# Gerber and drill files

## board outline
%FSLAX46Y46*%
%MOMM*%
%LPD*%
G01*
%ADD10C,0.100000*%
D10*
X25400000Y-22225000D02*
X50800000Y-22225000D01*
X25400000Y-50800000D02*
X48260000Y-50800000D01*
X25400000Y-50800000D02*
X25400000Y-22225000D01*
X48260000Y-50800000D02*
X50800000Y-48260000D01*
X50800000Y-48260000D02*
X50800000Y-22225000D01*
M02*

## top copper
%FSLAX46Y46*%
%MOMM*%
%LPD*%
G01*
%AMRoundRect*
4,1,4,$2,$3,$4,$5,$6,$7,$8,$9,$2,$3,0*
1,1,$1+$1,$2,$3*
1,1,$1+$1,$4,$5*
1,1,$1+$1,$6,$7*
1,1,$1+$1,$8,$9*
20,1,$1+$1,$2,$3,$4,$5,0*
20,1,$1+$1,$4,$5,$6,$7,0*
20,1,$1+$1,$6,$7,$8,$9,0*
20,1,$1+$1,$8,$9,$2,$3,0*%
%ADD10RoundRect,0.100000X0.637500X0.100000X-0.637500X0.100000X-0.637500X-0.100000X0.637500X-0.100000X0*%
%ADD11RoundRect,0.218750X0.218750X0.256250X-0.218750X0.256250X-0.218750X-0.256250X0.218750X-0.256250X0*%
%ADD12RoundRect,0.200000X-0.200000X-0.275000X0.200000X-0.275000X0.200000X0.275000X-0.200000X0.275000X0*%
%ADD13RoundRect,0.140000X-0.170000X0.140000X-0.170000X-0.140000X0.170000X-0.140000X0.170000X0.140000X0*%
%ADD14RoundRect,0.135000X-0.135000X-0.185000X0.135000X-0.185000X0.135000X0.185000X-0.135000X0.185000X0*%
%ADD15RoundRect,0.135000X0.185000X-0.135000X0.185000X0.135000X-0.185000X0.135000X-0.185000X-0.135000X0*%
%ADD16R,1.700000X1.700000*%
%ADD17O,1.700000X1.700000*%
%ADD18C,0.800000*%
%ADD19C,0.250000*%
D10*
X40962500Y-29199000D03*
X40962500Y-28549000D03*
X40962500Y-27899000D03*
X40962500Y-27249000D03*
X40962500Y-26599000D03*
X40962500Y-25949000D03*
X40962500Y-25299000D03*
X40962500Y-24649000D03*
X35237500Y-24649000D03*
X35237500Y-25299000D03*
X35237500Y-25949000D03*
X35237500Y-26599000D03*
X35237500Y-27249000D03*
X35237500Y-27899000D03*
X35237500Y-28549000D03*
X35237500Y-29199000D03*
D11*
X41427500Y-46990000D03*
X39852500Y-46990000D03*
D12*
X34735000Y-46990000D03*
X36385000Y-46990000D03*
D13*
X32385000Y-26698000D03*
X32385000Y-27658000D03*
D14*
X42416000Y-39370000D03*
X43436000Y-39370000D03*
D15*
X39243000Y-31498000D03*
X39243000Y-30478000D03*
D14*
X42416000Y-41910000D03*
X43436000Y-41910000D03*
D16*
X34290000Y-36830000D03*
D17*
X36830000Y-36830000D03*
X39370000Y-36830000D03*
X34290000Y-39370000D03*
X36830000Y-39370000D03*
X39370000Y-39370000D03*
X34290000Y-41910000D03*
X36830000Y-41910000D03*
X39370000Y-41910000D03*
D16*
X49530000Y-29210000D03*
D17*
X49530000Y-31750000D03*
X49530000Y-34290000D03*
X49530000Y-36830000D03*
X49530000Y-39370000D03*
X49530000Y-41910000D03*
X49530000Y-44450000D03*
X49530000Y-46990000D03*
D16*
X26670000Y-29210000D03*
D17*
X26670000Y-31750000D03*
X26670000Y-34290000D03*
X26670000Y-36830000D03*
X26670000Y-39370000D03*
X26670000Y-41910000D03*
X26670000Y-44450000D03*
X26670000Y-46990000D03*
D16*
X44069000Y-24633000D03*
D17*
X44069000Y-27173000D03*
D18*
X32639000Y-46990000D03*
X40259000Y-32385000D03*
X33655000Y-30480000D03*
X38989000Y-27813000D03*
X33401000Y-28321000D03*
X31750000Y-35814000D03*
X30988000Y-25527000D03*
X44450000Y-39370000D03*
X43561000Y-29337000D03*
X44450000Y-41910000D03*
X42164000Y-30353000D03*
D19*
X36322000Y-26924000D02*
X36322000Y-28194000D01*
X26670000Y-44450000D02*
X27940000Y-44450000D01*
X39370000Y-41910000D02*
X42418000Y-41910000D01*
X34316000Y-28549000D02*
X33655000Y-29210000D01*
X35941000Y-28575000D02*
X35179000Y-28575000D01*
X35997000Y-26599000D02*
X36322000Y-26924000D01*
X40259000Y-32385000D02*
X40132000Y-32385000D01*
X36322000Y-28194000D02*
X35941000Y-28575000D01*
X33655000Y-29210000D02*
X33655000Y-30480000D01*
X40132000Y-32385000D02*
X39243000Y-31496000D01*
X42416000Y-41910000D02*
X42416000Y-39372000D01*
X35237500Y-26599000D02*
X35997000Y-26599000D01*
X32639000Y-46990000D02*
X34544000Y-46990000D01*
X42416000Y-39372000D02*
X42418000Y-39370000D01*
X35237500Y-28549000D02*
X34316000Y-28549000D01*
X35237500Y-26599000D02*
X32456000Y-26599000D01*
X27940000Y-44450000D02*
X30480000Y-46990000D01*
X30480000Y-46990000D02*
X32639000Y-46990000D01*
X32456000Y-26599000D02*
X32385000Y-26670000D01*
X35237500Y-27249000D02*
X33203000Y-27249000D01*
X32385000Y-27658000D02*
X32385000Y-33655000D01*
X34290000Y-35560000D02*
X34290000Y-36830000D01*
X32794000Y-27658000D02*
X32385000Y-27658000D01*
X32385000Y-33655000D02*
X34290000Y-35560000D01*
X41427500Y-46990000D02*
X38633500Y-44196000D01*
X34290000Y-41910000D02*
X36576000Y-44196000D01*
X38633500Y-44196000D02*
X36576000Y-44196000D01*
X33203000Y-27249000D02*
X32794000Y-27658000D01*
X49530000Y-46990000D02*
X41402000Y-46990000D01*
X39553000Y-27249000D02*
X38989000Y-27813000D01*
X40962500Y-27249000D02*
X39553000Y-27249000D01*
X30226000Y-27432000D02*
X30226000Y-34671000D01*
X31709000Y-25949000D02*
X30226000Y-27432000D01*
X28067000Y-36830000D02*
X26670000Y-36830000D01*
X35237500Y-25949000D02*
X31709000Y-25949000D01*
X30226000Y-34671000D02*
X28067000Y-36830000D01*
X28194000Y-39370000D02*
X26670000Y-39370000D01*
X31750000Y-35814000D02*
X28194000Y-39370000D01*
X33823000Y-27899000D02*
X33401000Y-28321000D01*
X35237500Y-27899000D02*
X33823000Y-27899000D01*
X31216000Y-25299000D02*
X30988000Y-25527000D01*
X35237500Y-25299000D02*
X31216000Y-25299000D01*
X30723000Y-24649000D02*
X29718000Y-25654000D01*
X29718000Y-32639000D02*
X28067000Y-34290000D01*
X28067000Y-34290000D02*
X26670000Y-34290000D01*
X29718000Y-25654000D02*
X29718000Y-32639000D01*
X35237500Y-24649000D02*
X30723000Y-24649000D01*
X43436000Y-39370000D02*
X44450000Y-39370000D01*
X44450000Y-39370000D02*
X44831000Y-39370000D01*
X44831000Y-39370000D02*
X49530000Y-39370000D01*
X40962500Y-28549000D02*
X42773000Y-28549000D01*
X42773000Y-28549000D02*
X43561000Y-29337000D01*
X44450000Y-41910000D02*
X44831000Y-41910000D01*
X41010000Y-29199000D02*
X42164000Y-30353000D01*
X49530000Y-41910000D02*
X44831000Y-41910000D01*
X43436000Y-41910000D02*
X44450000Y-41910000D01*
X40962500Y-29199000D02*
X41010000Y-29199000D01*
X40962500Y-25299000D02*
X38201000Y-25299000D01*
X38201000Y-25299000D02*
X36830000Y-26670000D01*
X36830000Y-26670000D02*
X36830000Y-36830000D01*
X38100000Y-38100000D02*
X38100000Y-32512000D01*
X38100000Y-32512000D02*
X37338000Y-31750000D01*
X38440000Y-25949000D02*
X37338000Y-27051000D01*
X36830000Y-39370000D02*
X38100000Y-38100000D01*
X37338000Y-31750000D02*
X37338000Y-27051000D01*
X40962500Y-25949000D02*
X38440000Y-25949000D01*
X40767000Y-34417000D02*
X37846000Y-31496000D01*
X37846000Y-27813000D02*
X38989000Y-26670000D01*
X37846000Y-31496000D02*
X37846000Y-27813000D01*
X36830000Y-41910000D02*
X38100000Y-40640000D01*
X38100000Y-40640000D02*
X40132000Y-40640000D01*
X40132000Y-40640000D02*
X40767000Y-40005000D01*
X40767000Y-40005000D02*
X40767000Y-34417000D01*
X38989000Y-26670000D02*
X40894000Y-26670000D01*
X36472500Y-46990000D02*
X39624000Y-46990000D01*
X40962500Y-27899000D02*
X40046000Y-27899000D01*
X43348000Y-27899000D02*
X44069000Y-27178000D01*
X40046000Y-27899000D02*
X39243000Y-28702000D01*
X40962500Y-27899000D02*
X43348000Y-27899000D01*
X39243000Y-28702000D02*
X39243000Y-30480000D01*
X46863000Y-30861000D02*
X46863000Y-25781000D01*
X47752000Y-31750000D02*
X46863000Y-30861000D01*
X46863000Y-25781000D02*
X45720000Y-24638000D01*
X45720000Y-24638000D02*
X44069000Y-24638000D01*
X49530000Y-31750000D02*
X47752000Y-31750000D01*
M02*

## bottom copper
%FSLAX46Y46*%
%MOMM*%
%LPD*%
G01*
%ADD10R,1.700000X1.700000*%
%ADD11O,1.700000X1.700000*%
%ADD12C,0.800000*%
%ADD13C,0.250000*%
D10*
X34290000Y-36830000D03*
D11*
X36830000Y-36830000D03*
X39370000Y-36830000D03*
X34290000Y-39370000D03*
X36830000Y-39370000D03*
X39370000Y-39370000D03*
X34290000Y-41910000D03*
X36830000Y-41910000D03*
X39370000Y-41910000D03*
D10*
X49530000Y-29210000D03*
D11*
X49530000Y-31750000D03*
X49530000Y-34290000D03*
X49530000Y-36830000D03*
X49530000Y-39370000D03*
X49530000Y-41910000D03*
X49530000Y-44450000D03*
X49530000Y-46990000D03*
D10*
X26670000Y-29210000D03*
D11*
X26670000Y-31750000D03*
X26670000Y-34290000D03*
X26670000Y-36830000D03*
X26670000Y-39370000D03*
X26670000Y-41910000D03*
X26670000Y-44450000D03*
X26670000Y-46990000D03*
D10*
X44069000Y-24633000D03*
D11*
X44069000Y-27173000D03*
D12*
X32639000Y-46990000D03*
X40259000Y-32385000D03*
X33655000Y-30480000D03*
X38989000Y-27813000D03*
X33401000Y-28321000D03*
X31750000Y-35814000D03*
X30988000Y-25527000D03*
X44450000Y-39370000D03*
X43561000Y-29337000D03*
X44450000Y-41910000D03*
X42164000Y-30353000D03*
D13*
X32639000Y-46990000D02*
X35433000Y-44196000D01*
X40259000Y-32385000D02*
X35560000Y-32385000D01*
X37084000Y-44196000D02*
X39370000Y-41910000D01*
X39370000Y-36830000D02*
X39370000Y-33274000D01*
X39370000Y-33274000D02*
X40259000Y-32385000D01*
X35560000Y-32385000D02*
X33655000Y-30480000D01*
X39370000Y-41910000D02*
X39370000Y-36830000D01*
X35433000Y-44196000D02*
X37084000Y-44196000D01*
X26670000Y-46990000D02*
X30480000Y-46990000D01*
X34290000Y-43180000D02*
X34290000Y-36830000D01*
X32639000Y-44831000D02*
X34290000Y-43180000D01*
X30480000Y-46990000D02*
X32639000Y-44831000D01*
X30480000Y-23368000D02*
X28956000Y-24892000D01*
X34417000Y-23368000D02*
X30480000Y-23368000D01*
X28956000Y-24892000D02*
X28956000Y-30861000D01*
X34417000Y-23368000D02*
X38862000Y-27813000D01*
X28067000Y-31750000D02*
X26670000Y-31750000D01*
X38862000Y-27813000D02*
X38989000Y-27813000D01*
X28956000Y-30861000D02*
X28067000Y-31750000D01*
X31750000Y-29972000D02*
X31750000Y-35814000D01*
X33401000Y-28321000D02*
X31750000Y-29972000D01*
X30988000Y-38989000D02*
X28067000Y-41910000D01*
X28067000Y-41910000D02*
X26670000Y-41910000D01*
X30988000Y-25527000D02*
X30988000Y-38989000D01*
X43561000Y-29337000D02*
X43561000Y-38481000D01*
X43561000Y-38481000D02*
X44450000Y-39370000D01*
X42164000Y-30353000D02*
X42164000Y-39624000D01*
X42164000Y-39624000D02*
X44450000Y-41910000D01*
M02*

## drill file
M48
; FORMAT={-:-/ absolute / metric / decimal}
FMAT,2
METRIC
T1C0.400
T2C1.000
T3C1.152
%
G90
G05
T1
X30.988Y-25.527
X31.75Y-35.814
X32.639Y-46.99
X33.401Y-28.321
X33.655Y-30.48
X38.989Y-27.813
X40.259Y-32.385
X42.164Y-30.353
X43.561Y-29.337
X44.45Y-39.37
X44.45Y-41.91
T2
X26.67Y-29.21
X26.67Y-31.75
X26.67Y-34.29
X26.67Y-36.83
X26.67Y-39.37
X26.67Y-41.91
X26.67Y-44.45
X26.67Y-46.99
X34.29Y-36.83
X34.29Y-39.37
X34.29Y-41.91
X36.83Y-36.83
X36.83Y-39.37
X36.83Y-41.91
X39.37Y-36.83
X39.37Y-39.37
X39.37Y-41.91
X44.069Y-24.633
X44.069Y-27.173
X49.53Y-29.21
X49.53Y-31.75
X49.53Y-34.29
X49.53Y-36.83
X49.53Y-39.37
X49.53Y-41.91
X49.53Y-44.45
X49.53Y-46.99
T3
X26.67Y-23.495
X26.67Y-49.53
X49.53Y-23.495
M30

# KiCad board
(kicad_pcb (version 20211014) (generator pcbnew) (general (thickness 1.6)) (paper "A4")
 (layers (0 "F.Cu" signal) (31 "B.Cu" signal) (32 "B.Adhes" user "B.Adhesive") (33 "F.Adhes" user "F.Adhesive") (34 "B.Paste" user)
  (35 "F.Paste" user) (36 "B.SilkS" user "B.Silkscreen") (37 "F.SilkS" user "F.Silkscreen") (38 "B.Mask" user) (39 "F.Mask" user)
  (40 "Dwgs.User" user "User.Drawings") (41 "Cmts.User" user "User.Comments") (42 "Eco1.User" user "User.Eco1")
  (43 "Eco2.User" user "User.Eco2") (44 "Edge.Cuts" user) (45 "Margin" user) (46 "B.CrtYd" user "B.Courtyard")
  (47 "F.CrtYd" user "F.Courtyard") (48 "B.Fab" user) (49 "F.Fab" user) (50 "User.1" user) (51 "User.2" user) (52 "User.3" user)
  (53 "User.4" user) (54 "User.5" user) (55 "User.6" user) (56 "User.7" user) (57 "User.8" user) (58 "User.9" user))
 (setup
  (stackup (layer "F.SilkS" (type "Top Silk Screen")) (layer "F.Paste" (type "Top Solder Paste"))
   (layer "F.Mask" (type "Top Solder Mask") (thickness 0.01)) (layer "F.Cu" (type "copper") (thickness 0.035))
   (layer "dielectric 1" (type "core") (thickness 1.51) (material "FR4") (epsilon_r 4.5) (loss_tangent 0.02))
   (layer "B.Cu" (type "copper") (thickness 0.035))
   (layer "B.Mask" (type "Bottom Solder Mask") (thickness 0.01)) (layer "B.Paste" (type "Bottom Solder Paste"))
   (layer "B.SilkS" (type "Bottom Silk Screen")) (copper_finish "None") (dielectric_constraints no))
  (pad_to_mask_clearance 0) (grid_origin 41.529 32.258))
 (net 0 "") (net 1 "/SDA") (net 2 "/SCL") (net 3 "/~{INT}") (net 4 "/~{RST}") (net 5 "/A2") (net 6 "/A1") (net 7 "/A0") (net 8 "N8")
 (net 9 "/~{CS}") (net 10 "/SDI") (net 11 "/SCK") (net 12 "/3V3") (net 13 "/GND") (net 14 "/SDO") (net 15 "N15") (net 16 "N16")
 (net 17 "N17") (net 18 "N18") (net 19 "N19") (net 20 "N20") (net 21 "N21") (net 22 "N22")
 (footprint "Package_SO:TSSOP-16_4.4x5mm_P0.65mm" (layer "F.Cu") (at 38.1 26.924 180)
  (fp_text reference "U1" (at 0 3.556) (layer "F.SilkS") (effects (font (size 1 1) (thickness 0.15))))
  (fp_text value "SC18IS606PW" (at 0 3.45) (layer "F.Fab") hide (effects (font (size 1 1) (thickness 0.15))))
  (pad "1" smd roundrect (at -2.8625 -2.275 180) (size 1.475 0.4) (layers "F.Cu" "F.Paste" "F.Mask") (roundrect_rratio 0.25) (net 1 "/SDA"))
  (pad "2" smd roundrect (at -2.8625 -1.625 180) (size 1.475 0.4) (layers "F.Cu" "F.Paste" "F.Mask") (roundrect_rratio 0.25) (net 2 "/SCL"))
  (pad "3" smd roundrect (at -2.8625 -0.975 180) (size 1.475 0.4) (layers "F.Cu" "F.Paste" "F.Mask") (roundrect_rratio 0.25)
   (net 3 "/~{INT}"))
  (pad "4" smd roundrect (at -2.8625 -0.325 180) (size 1.475 0.4) (layers "F.Cu" "F.Paste" "F.Mask") (roundrect_rratio 0.25)
   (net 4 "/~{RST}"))
  (pad "5" smd roundrect (at -2.8625 0.325 180) (size 1.475 0.4) (layers "F.Cu" "F.Paste" "F.Mask") (roundrect_rratio 0.25) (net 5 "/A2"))
  (pad "6" smd roundrect (at -2.8625 0.975 180) (size 1.475 0.4) (layers "F.Cu" "F.Paste" "F.Mask") (roundrect_rratio 0.25) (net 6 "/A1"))
  (pad "7" smd roundrect (at -2.8625 1.625 180) (size 1.475 0.4) (layers "F.Cu" "F.Paste" "F.Mask") (roundrect_rratio 0.25) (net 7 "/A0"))
  (pad "8" smd roundrect (at -2.8625 2.275 180) (size 1.475 0.4) (layers "F.Cu" "F.Paste" "F.Mask") (roundrect_rratio 0.25) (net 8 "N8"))
  (pad "9" smd roundrect (at 2.8625 2.275 180) (size 1.475 0.4) (layers "F.Cu" "F.Paste" "F.Mask") (roundrect_rratio 0.25) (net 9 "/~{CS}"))
  (pad "10" smd roundrect (at 2.8625 1.625 180) (size 1.475 0.4) (layers "F.Cu" "F.Paste" "F.Mask") (roundrect_rratio 0.25) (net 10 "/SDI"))
  (pad "11" smd roundrect (at 2.8625 0.975 180) (size 1.475 0.4) (layers "F.Cu" "F.Paste" "F.Mask") (roundrect_rratio 0.25) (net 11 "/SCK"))
  (pad "12" smd roundrect (at 2.8625 0.325 180) (size 1.475 0.4) (layers "F.Cu" "F.Paste" "F.Mask") (roundrect_rratio 0.25) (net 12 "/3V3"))
  (pad "13" smd roundrect (at 2.8625 -0.325 180) (size 1.475 0.4) (layers "F.Cu" "F.Paste" "F.Mask") (roundrect_rratio 0.25) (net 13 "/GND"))
  (pad "14" smd roundrect (at 2.8625 -0.975 180) (size 1.475 0.4) (layers "F.Cu" "F.Paste" "F.Mask") (roundrect_rratio 0.25) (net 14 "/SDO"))
  (pad "15" smd roundrect (at 2.8625 -1.625 180) (size 1.475 0.4) (layers "F.Cu" "F.Paste" "F.Mask") (roundrect_rratio 0.25) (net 12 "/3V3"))
  (pad "16" smd roundrect (at 2.8625 -2.275 180) (size 1.475 0.4) (layers "F.Cu" "F.Paste" "F.Mask") (roundrect_rratio 0.25) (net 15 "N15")))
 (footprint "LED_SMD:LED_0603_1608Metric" (layer "F.Cu") (at 40.64 46.99 180)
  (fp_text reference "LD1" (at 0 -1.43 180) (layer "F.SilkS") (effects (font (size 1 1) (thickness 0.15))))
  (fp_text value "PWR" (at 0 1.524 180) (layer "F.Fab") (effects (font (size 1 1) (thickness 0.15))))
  (pad "1" smd roundrect (at -0.7875 0 180) (size 0.875 0.95) (layers "F.Cu" "F.Paste" "F.Mask") (roundrect_rratio 0.25) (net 13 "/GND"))
  (pad "2" smd roundrect (at 0.7875 0 180) (size 0.875 0.95) (layers "F.Cu" "F.Paste" "F.Mask") (roundrect_rratio 0.25) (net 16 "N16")))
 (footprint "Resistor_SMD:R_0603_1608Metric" (layer "F.Cu") (at 35.56 46.99)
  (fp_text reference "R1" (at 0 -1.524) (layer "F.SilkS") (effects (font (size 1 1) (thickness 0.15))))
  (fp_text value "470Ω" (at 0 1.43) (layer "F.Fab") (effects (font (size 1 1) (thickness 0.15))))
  (pad "1" smd roundrect (at -0.825 0) (size 0.8 0.95) (layers "F.Cu" "F.Paste" "F.Mask") (roundrect_rratio 0.25) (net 12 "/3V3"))
  (pad "2" smd roundrect (at 0.825 0) (size 0.8 0.95) (layers "F.Cu" "F.Paste" "F.Mask") (roundrect_rratio 0.25) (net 16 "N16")))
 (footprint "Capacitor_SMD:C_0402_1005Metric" (layer "F.Cu") (at 32.385 27.178 -90)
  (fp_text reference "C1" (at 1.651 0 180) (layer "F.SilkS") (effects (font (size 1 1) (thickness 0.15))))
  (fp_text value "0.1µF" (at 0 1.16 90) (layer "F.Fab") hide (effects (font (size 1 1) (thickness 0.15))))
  (pad "1" smd roundrect (at -0.48 0 270) (size 0.56 0.62) (layers "F.Cu" "F.Paste" "F.Mask") (roundrect_rratio 0.25) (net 12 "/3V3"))
  (pad "2" smd roundrect (at 0.48 0 270) (size 0.56 0.62) (layers "F.Cu" "F.Paste" "F.Mask") (roundrect_rratio 0.25) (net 13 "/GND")))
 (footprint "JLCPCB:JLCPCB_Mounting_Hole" (layer "F.Cu") (at 26.67 23.495)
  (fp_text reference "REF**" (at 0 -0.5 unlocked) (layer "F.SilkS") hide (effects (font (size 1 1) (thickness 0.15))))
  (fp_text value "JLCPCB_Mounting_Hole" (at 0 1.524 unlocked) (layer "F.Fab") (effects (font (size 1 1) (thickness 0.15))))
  (pad "" np_thru_hole circle (at 0 0) (size 1.152 1.152) (drill 1.152) (layers F&B.Cu *.Mask) (solder_mask_margin 0.148)))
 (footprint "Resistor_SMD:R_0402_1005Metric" (layer "F.Cu") (at 42.926 39.37)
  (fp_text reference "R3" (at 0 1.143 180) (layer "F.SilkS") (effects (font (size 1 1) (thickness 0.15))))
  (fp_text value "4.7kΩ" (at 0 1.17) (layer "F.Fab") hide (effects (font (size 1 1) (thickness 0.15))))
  (pad "1" smd roundrect (at -0.51 0) (size 0.54 0.64) (layers "F.Cu" "F.Paste" "F.Mask") (roundrect_rratio 0.25) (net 12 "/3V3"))
  (pad "2" smd roundrect (at 0.51 0) (size 0.54 0.64) (layers "F.Cu" "F.Paste" "F.Mask") (roundrect_rratio 0.25) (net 2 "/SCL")))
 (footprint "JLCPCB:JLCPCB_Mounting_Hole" (layer "F.Cu") (at 26.67 49.53)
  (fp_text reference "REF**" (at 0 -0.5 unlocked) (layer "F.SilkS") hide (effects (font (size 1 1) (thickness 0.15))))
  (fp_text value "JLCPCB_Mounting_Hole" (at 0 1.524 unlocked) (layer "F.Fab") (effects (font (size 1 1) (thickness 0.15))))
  (pad "" np_thru_hole circle (at 0 0) (size 1.152 1.152) (drill 1.152) (layers F&B.Cu *.Mask) (solder_mask_margin 0.148)))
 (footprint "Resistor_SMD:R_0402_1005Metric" (layer "F.Cu") (at 39.243 30.988 90)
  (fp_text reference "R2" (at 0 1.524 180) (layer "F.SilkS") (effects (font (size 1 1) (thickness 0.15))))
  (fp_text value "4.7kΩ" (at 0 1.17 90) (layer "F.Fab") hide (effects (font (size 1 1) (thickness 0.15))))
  (pad "1" smd roundrect (at -0.51 0 90) (size 0.54 0.64) (layers "F.Cu" "F.Paste" "F.Mask") (roundrect_rratio 0.25) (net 12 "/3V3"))
  (pad "2" smd roundrect (at 0.51 0 90) (size 0.54 0.64) (layers "F.Cu" "F.Paste" "F.Mask") (roundrect_rratio 0.25) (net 3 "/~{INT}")))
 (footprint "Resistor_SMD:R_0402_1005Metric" (layer "F.Cu") (at 42.926 41.91)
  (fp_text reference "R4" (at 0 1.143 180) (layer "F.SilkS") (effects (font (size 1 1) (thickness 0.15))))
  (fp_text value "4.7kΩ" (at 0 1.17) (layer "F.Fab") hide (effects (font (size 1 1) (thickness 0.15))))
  (pad "1" smd roundrect (at -0.51 0) (size 0.54 0.64) (layers "F.Cu" "F.Paste" "F.Mask") (roundrect_rratio 0.25) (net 12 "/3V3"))
  (pad "2" smd roundrect (at 0.51 0) (size 0.54 0.64) (layers "F.Cu" "F.Paste" "F.Mask") (roundrect_rratio 0.25) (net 1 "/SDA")))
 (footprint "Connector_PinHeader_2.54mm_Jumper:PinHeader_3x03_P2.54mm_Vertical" (layer "F.Cu") (at 34.29 36.83)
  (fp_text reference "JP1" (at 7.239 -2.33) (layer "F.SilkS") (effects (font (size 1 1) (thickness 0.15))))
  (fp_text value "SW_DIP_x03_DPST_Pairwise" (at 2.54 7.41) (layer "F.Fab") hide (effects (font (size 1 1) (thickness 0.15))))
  (pad "1" thru_hole rect (at 0 0) (size 1.7 1.7) (drill 1) (layers *.Cu *.Mask) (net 13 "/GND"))
  (pad "2" thru_hole oval (at 2.54 0) (size 1.7 1.7) (drill 1) (layers *.Cu *.Mask) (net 7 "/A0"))
  (pad "3" thru_hole oval (at 5.08 0) (size 1.7 1.7) (drill 1) (layers *.Cu *.Mask) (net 12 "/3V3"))
  (pad "4" thru_hole oval (at 0 2.54) (size 1.7 1.7) (drill 1) (layers *.Cu *.Mask) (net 13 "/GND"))
  (pad "5" thru_hole oval (at 2.54 2.54) (size 1.7 1.7) (drill 1) (layers *.Cu *.Mask) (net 6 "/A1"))
  (pad "6" thru_hole oval (at 5.08 2.54) (size 1.7 1.7) (drill 1) (layers *.Cu *.Mask) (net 12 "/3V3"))
  (pad "7" thru_hole oval (at 0 5.08) (size 1.7 1.7) (drill 1) (layers *.Cu *.Mask) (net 13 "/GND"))
  (pad "8" thru_hole oval (at 2.54 5.08) (size 1.7 1.7) (drill 1) (layers *.Cu *.Mask) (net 5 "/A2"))
  (pad "9" thru_hole oval (at 5.08 5.08) (size 1.7 1.7) (drill 1) (layers *.Cu *.Mask) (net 12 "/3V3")))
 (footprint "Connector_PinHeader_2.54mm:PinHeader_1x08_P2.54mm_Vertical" (layer "F.Cu") (at 49.53 29.21)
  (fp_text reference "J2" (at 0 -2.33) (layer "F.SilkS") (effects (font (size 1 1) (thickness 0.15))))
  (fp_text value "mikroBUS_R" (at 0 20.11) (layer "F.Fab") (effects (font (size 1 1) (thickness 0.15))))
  (pad "1" thru_hole rect (at 0 0) (size 1.7 1.7) (drill 1) (layers *.Cu *.Mask) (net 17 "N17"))
  (pad "2" thru_hole oval (at 0 2.54) (size 1.7 1.7) (drill 1) (layers *.Cu *.Mask) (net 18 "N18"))
  (pad "3" thru_hole oval (at 0 5.08) (size 1.7 1.7) (drill 1) (layers *.Cu *.Mask) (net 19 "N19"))
  (pad "4" thru_hole oval (at 0 7.62) (size 1.7 1.7) (drill 1) (layers *.Cu *.Mask) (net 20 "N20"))
  (pad "5" thru_hole oval (at 0 10.16) (size 1.7 1.7) (drill 1) (layers *.Cu *.Mask) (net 2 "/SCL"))
  (pad "6" thru_hole oval (at 0 12.7) (size 1.7 1.7) (drill 1) (layers *.Cu *.Mask) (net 1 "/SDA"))
  (pad "7" thru_hole oval (at 0 15.24) (size 1.7 1.7) (drill 1) (layers *.Cu *.Mask) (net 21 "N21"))
  (pad "8" thru_hole oval (at 0 17.78) (size 1.7 1.7) (drill 1) (layers *.Cu *.Mask) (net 13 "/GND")))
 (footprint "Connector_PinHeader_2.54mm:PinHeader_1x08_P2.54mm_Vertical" (layer "F.Cu") (at 26.67 29.21)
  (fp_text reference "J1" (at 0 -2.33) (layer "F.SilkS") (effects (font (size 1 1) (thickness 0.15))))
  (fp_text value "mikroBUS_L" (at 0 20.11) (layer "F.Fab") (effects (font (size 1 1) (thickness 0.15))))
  (pad "1" thru_hole rect (at 0 0) (size 1.7 1.7) (drill 1) (layers *.Cu *.Mask) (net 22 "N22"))
  (pad "2" thru_hole oval (at 0 2.54) (size 1.7 1.7) (drill 1) (layers *.Cu *.Mask) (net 4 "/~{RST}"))
  (pad "3" thru_hole oval (at 0 5.08) (size 1.7 1.7) (drill 1) (layers *.Cu *.Mask) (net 9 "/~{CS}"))
  (pad "4" thru_hole oval (at 0 7.62) (size 1.7 1.7) (drill 1) (layers *.Cu *.Mask) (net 11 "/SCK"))
  (pad "5" thru_hole oval (at 0 10.16) (size 1.7 1.7) (drill 1) (layers *.Cu *.Mask) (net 14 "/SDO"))
  (pad "6" thru_hole oval (at 0 12.7) (size 1.7 1.7) (drill 1) (layers *.Cu *.Mask) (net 10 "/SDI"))
  (pad "7" thru_hole oval (at 0 15.24) (size 1.7 1.7) (drill 1) (layers *.Cu *.Mask) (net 12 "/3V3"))
  (pad "8" thru_hole oval (at 0 17.78) (size 1.7 1.7) (drill 1) (layers *.Cu *.Mask) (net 13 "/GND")))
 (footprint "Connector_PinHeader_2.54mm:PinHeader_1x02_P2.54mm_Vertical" (layer "F.Cu") (at 44.069 24.633)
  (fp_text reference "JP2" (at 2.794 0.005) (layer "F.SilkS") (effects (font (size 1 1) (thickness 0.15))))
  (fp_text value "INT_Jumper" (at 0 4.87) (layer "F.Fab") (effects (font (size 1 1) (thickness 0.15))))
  (pad "1" thru_hole rect (at 0 0) (size 1.7 1.7) (drill 1) (layers *.Cu *.Mask) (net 18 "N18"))
  (pad "2" thru_hole oval (at 0 2.54) (size 1.7 1.7) (drill 1) (layers *.Cu *.Mask) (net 3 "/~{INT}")))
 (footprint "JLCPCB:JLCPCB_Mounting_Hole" (layer "F.Cu") (at 49.53 23.495)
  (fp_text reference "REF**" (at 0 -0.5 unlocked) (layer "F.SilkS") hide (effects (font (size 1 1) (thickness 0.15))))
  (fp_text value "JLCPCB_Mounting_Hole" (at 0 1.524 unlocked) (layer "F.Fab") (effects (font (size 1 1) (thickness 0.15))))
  (pad "" np_thru_hole circle (at 0 0) (size 1.152 1.152) (drill 1.152) (layers F&B.Cu *.Mask) (solder_mask_margin 0.148)))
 (gr_line (start 25.4 22.225) (end 50.8 22.225) (layer "Edge.Cuts") (width 0.1))
 (gr_line (start 25.4 50.8) (end 48.26 50.8) (layer "Edge.Cuts") (width 0.1))
 (gr_line (start 25.4 50.8) (end 25.4 22.225) (layer "Edge.Cuts") (width 0.1))
 (gr_line (start 48.26 50.8) (end 50.8 48.26) (layer "Edge.Cuts") (width 0.1))
 (gr_line (start 50.8 48.26) (end 50.8 22.225) (layer "Edge.Cuts") (width 0.1))
 (segment (start 36.322 26.924) (end 36.322 28.194) (width 0.25) (layer "F.Cu") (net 12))
 (segment (start 26.67 44.45) (end 27.94 44.45) (width 0.25) (layer "F.Cu") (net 12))
 (segment (start 39.37 41.91) (end 42.418 41.91) (width 0.25) (layer "F.Cu") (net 12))
 (segment (start 34.316 28.549) (end 33.655 29.21) (width 0.25) (layer "F.Cu") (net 12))
 (segment (start 35.941 28.575) (end 35.179 28.575) (width 0.25) (layer "F.Cu") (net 12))
 (segment (start 35.997 26.599) (end 36.322 26.924) (width 0.25) (layer "F.Cu") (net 12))
 (segment (start 40.259 32.385) (end 40.132 32.385) (width 0.25) (layer "F.Cu") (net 12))
 (segment (start 36.322 28.194) (end 35.941 28.575) (width 0.25) (layer "F.Cu") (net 12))
 (segment (start 33.655 29.21) (end 33.655 30.48) (width 0.25) (layer "F.Cu") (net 12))
 (segment (start 40.132 32.385) (end 39.243 31.496) (width 0.25) (layer "F.Cu") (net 12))
 (segment (start 42.416 41.91) (end 42.416 39.372) (width 0.25) (layer "F.Cu") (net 12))
 (segment (start 35.2375 26.599) (end 35.997 26.599) (width 0.25) (layer "F.Cu") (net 12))
 (segment (start 32.639 46.99) (end 34.544 46.99) (width 0.25) (layer "F.Cu") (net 12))
 (segment (start 42.416 39.372) (end 42.418 39.37) (width 0.25) (layer "F.Cu") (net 12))
 (segment (start 35.2375 28.549) (end 34.316 28.549) (width 0.25) (layer "F.Cu") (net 12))
 (segment (start 35.2375 26.599) (end 32.456 26.599) (width 0.25) (layer "F.Cu") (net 12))
 (segment (start 27.94 44.45) (end 30.48 46.99) (width 0.25) (layer "F.Cu") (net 12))
 (segment (start 30.48 46.99) (end 32.639 46.99) (width 0.25) (layer "F.Cu") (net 12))
 (segment (start 32.456 26.599) (end 32.385 26.67) (width 0.25) (layer "F.Cu") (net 12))
 (via (at 32.639 46.99) (size 0.8) (drill 0.4) (layers "F.Cu" "B.Cu") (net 12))
 (via (at 40.259 32.385) (size 0.8) (drill 0.4) (layers "F.Cu" "B.Cu") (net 12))
 (via (at 33.655 30.48) (size 0.8) (drill 0.4) (layers "F.Cu" "B.Cu") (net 12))
 (segment (start 32.639 46.99) (end 35.433 44.196) (width 0.25) (layer "B.Cu") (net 12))
 (segment (start 40.259 32.385) (end 35.56 32.385) (width 0.25) (layer "B.Cu") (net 12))
 (segment (start 37.084 44.196) (end 39.37 41.91) (width 0.25) (layer "B.Cu") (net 12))
 (segment (start 39.37 36.83) (end 39.37 33.274) (width 0.25) (layer "B.Cu") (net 12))
 (segment (start 39.37 33.274) (end 40.259 32.385) (width 0.25) (layer "B.Cu") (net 12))
 (segment (start 35.56 32.385) (end 33.655 30.48) (width 0.25) (layer "B.Cu") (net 12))
 (segment (start 39.37 41.91) (end 39.37 36.83) (width 0.25) (layer "B.Cu") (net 12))
 (segment (start 35.433 44.196) (end 37.084 44.196) (width 0.25) (layer "B.Cu") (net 12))
 (segment (start 35.2375 27.249) (end 33.203 27.249) (width 0.25) (layer "F.Cu") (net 13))
 (segment (start 32.385 27.658) (end 32.385 33.655) (width 0.25) (layer "F.Cu") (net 13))
 (segment (start 34.29 35.56) (end 34.29 36.83) (width 0.25) (layer "F.Cu") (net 13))
 (segment (start 32.794 27.658) (end 32.385 27.658) (width 0.25) (layer "F.Cu") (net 13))
 (segment (start 32.385 33.655) (end 34.29 35.56) (width 0.25) (layer "F.Cu") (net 13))
 (segment (start 41.4275 46.99) (end 38.6335 44.196) (width 0.25) (layer "F.Cu") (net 13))
 (segment (start 34.29 41.91) (end 36.576 44.196) (width 0.25) (layer "F.Cu") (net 13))
 (segment (start 38.6335 44.196) (end 36.576 44.196) (width 0.25) (layer "F.Cu") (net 13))
 (segment (start 33.203 27.249) (end 32.794 27.658) (width 0.25) (layer "F.Cu") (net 13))
 (segment (start 49.53 46.99) (end 41.402 46.99) (width 0.25) (layer "F.Cu") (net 13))
 (segment (start 26.67 46.99) (end 30.48 46.99) (width 0.25) (layer "B.Cu") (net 13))
 (segment (start 34.29 43.18) (end 34.29 36.83) (width 0.25) (layer "B.Cu") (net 13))
 (segment (start 32.639 44.831) (end 34.29 43.18) (width 0.25) (layer "B.Cu") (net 13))
 (segment (start 30.48 46.99) (end 32.639 44.831) (width 0.25) (layer "B.Cu") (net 13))
 (segment (start 39.553 27.249) (end 38.989 27.813) (width 0.25) (layer "F.Cu") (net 4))
 (segment (start 40.9625 27.249) (end 39.553 27.249) (width 0.25) (layer "F.Cu") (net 4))
 (via (at 38.989 27.813) (size 0.8) (drill 0.4) (layers "F.Cu" "B.Cu") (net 4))
 (segment (start 30.48 23.368) (end 28.956 24.892) (width 0.25) (layer "B.Cu") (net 4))
 (segment (start 34.417 23.368) (end 30.48 23.368) (width 0.25) (layer "B.Cu") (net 4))
 (segment (start 28.956 24.892) (end 28.956 30.861) (width 0.25) (layer "B.Cu") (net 4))
 (segment (start 34.417 23.368) (end 38.862 27.813) (width 0.25) (layer "B.Cu") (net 4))
 (segment (start 28.067 31.75) (end 26.67 31.75) (width 0.25) (layer "B.Cu") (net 4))
 (segment (start 38.862 27.813) (end 38.989 27.813) (width 0.25) (layer "B.Cu") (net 4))
 (segment (start 28.956 30.861) (end 28.067 31.75) (width 0.25) (layer "B.Cu") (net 4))
 (segment (start 30.226 27.432) (end 30.226 34.671) (width 0.25) (layer "F.Cu") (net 11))
 (segment (start 31.709 25.949) (end 30.226 27.432) (width 0.25) (layer "F.Cu") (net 11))
 (segment (start 28.067 36.83) (end 26.67 36.83) (width 0.25) (layer "F.Cu") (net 11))
 (segment (start 35.2375 25.949) (end 31.709 25.949) (width 0.25) (layer "F.Cu") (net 11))
 (segment (start 30.226 34.671) (end 28.067 36.83) (width 0.25) (layer "F.Cu") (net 11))
 (segment (start 28.194 39.37) (end 26.67 39.37) (width 0.25) (layer "F.Cu") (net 14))
 (segment (start 31.75 35.814) (end 28.194 39.37) (width 0.25) (layer "F.Cu") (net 14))
 (segment (start 33.823 27.899) (end 33.401 28.321) (width 0.25) (layer "F.Cu") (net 14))
 (segment (start 35.2375 27.899) (end 33.823 27.899) (width 0.25) (layer "F.Cu") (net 14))
 (via (at 33.401 28.321) (size 0.8) (drill 0.4) (layers "F.Cu" "B.Cu") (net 14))
 (via (at 31.75 35.814) (size 0.8) (drill 0.4) (layers "F.Cu" "B.Cu") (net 14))
 (segment (start 31.75 29.972) (end 31.75 35.814) (width 0.25) (layer "B.Cu") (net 14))
 (segment (start 33.401 28.321) (end 31.75 29.972) (width 0.25) (layer "B.Cu") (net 14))
 (segment (start 31.216 25.299) (end 30.988 25.527) (width 0.25) (layer "F.Cu") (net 10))
 (segment (start 35.2375 25.299) (end 31.216 25.299) (width 0.25) (layer "F.Cu") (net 10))
 (via (at 30.988 25.527) (size 0.8) (drill 0.4) (layers "F.Cu" "B.Cu") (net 10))
 (segment (start 30.988 38.989) (end 28.067 41.91) (width 0.25) (layer "B.Cu") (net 10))
 (segment (start 28.067 41.91) (end 26.67 41.91) (width 0.25) (layer "B.Cu") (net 10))
 (segment (start 30.988 25.527) (end 30.988 38.989) (width 0.25) (layer "B.Cu") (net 10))
 (segment (start 30.723 24.649) (end 29.718 25.654) (width 0.25) (layer "F.Cu") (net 9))
 (segment (start 29.718 32.639) (end 28.067 34.29) (width 0.25) (layer "F.Cu") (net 9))
 (segment (start 28.067 34.29) (end 26.67 34.29) (width 0.25) (layer "F.Cu") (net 9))
 (segment (start 29.718 25.654) (end 29.718 32.639) (width 0.25) (layer "F.Cu") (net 9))
 (segment (start 35.2375 24.649) (end 30.723 24.649) (width 0.25) (layer "F.Cu") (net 9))
 (segment (start 43.436 39.37) (end 44.45 39.37) (width 0.25) (layer "F.Cu") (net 2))
 (segment (start 44.45 39.37) (end 44.831 39.37) (width 0.25) (layer "F.Cu") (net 2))
 (segment (start 44.831 39.37) (end 49.53 39.37) (width 0.25) (layer "F.Cu") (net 2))
 (segment (start 40.9625 28.549) (end 42.773 28.549) (width 0.25) (layer "F.Cu") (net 2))
 (segment (start 42.773 28.549) (end 43.561 29.337) (width 0.25) (layer "F.Cu") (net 2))
 (via (at 44.45 39.37) (size 0.8) (drill 0.4) (layers "F.Cu" "B.Cu") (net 2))
 (via (at 43.561 29.337) (size 0.8) (drill 0.4) (layers "F.Cu" "B.Cu") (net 2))
 (segment (start 43.561 29.337) (end 43.561 38.481) (width 0.25) (layer "B.Cu") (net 2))
 (segment (start 43.561 38.481) (end 44.45 39.37) (width 0.25) (layer "B.Cu") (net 2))
 (segment (start 44.45 41.91) (end 44.831 41.91) (width 0.25) (layer "F.Cu") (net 1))
 (segment (start 41.01 29.199) (end 42.164 30.353) (width 0.25) (layer "F.Cu") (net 1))
 (segment (start 49.53 41.91) (end 44.831 41.91) (width 0.25) (layer "F.Cu") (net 1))
 (segment (start 43.436 41.91) (end 44.45 41.91) (width 0.25) (layer "F.Cu") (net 1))
 (segment (start 40.9625 29.199) (end 41.01 29.199) (width 0.25) (layer "F.Cu") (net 1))
 (via (at 44.45 41.91) (size 0.8) (drill 0.4) (layers "F.Cu" "B.Cu") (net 1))
 (via (at 42.164 30.353) (size 0.8) (drill 0.4) (layers "F.Cu" "B.Cu") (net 1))
 (segment (start 42.164 30.353) (end 42.164 39.624) (width 0.25) (layer "B.Cu") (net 1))
 (segment (start 42.164 39.624) (end 44.45 41.91) (width 0.25) (layer "B.Cu") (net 1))
 (segment (start 40.9625 25.299) (end 38.201 25.299) (width 0.25) (layer "F.Cu") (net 7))
 (segment (start 38.201 25.299) (end 36.83 26.67) (width 0.25) (layer "F.Cu") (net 7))
 (segment (start 36.83 26.67) (end 36.83 36.83) (width 0.25) (layer "F.Cu") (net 7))
 (segment (start 38.1 38.1) (end 38.1 32.512) (width 0.25) (layer "F.Cu") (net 6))
 (segment (start 38.1 32.512) (end 37.338 31.75) (width 0.25) (layer "F.Cu") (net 6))
 (segment (start 38.44 25.949) (end 37.338 27.051) (width 0.25) (layer "F.Cu") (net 6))
 (segment (start 36.83 39.37) (end 38.1 38.1) (width 0.25) (layer "F.Cu") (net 6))
 (segment (start 37.338 31.75) (end 37.338 27.051) (width 0.25) (layer "F.Cu") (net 6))
 (segment (start 40.9625 25.949) (end 38.44 25.949) (width 0.25) (layer "F.Cu") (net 6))
 (segment (start 40.767 34.417) (end 37.846 31.496) (width 0.25) (layer "F.Cu") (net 5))
 (segment (start 37.846 27.813) (end 38.989 26.67) (width 0.25) (layer "F.Cu") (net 5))
 (segment (start 37.846 31.496) (end 37.846 27.813) (width 0.25) (layer "F.Cu") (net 5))
 (segment (start 36.83 41.91) (end 38.1 40.64) (width 0.25) (layer "F.Cu") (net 5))
 (segment (start 38.1 40.64) (end 40.132 40.64) (width 0.25) (layer "F.Cu") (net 5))
 (segment (start 40.132 40.64) (end 40.767 40.005) (width 0.25) (layer "F.Cu") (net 5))
 (segment (start 40.767 40.005) (end 40.767 34.417) (width 0.25) (layer "F.Cu") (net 5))
 (segment (start 38.989 26.67) (end 40.894 26.67) (width 0.25) (layer "F.Cu") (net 5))
 (segment (start 36.4725 46.99) (end 39.624 46.99) (width 0.25) (layer "F.Cu") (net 16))
 (segment (start 40.9625 27.899) (end 40.046 27.899) (width 0.25) (layer "F.Cu") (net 3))
 (segment (start 43.348 27.899) (end 44.069 27.178) (width 0.25) (layer "F.Cu") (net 3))
 (segment (start 40.046 27.899) (end 39.243 28.702) (width 0.25) (layer "F.Cu") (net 3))
 (segment (start 40.9625 27.899) (end 43.348 27.899) (width 0.25) (layer "F.Cu") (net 3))
 (segment (start 39.243 28.702) (end 39.243 30.48) (width 0.25) (layer "F.Cu") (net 3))
 (segment (start 46.863 30.861) (end 46.863 25.781) (width 0.25) (layer "F.Cu") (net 18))
 (segment (start 47.752 31.75) (end 46.863 30.861) (width 0.25) (layer "F.Cu") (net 18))
 (segment (start 46.863 25.781) (end 45.72 24.638) (width 0.25) (layer "F.Cu") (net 18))
 (segment (start 45.72 24.638) (end 44.069 24.638) (width 0.25) (layer "F.Cu") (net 18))
 (segment (start 49.53 31.75) (end 47.752 31.75) (width 0.25) (layer "F.Cu") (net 18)))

